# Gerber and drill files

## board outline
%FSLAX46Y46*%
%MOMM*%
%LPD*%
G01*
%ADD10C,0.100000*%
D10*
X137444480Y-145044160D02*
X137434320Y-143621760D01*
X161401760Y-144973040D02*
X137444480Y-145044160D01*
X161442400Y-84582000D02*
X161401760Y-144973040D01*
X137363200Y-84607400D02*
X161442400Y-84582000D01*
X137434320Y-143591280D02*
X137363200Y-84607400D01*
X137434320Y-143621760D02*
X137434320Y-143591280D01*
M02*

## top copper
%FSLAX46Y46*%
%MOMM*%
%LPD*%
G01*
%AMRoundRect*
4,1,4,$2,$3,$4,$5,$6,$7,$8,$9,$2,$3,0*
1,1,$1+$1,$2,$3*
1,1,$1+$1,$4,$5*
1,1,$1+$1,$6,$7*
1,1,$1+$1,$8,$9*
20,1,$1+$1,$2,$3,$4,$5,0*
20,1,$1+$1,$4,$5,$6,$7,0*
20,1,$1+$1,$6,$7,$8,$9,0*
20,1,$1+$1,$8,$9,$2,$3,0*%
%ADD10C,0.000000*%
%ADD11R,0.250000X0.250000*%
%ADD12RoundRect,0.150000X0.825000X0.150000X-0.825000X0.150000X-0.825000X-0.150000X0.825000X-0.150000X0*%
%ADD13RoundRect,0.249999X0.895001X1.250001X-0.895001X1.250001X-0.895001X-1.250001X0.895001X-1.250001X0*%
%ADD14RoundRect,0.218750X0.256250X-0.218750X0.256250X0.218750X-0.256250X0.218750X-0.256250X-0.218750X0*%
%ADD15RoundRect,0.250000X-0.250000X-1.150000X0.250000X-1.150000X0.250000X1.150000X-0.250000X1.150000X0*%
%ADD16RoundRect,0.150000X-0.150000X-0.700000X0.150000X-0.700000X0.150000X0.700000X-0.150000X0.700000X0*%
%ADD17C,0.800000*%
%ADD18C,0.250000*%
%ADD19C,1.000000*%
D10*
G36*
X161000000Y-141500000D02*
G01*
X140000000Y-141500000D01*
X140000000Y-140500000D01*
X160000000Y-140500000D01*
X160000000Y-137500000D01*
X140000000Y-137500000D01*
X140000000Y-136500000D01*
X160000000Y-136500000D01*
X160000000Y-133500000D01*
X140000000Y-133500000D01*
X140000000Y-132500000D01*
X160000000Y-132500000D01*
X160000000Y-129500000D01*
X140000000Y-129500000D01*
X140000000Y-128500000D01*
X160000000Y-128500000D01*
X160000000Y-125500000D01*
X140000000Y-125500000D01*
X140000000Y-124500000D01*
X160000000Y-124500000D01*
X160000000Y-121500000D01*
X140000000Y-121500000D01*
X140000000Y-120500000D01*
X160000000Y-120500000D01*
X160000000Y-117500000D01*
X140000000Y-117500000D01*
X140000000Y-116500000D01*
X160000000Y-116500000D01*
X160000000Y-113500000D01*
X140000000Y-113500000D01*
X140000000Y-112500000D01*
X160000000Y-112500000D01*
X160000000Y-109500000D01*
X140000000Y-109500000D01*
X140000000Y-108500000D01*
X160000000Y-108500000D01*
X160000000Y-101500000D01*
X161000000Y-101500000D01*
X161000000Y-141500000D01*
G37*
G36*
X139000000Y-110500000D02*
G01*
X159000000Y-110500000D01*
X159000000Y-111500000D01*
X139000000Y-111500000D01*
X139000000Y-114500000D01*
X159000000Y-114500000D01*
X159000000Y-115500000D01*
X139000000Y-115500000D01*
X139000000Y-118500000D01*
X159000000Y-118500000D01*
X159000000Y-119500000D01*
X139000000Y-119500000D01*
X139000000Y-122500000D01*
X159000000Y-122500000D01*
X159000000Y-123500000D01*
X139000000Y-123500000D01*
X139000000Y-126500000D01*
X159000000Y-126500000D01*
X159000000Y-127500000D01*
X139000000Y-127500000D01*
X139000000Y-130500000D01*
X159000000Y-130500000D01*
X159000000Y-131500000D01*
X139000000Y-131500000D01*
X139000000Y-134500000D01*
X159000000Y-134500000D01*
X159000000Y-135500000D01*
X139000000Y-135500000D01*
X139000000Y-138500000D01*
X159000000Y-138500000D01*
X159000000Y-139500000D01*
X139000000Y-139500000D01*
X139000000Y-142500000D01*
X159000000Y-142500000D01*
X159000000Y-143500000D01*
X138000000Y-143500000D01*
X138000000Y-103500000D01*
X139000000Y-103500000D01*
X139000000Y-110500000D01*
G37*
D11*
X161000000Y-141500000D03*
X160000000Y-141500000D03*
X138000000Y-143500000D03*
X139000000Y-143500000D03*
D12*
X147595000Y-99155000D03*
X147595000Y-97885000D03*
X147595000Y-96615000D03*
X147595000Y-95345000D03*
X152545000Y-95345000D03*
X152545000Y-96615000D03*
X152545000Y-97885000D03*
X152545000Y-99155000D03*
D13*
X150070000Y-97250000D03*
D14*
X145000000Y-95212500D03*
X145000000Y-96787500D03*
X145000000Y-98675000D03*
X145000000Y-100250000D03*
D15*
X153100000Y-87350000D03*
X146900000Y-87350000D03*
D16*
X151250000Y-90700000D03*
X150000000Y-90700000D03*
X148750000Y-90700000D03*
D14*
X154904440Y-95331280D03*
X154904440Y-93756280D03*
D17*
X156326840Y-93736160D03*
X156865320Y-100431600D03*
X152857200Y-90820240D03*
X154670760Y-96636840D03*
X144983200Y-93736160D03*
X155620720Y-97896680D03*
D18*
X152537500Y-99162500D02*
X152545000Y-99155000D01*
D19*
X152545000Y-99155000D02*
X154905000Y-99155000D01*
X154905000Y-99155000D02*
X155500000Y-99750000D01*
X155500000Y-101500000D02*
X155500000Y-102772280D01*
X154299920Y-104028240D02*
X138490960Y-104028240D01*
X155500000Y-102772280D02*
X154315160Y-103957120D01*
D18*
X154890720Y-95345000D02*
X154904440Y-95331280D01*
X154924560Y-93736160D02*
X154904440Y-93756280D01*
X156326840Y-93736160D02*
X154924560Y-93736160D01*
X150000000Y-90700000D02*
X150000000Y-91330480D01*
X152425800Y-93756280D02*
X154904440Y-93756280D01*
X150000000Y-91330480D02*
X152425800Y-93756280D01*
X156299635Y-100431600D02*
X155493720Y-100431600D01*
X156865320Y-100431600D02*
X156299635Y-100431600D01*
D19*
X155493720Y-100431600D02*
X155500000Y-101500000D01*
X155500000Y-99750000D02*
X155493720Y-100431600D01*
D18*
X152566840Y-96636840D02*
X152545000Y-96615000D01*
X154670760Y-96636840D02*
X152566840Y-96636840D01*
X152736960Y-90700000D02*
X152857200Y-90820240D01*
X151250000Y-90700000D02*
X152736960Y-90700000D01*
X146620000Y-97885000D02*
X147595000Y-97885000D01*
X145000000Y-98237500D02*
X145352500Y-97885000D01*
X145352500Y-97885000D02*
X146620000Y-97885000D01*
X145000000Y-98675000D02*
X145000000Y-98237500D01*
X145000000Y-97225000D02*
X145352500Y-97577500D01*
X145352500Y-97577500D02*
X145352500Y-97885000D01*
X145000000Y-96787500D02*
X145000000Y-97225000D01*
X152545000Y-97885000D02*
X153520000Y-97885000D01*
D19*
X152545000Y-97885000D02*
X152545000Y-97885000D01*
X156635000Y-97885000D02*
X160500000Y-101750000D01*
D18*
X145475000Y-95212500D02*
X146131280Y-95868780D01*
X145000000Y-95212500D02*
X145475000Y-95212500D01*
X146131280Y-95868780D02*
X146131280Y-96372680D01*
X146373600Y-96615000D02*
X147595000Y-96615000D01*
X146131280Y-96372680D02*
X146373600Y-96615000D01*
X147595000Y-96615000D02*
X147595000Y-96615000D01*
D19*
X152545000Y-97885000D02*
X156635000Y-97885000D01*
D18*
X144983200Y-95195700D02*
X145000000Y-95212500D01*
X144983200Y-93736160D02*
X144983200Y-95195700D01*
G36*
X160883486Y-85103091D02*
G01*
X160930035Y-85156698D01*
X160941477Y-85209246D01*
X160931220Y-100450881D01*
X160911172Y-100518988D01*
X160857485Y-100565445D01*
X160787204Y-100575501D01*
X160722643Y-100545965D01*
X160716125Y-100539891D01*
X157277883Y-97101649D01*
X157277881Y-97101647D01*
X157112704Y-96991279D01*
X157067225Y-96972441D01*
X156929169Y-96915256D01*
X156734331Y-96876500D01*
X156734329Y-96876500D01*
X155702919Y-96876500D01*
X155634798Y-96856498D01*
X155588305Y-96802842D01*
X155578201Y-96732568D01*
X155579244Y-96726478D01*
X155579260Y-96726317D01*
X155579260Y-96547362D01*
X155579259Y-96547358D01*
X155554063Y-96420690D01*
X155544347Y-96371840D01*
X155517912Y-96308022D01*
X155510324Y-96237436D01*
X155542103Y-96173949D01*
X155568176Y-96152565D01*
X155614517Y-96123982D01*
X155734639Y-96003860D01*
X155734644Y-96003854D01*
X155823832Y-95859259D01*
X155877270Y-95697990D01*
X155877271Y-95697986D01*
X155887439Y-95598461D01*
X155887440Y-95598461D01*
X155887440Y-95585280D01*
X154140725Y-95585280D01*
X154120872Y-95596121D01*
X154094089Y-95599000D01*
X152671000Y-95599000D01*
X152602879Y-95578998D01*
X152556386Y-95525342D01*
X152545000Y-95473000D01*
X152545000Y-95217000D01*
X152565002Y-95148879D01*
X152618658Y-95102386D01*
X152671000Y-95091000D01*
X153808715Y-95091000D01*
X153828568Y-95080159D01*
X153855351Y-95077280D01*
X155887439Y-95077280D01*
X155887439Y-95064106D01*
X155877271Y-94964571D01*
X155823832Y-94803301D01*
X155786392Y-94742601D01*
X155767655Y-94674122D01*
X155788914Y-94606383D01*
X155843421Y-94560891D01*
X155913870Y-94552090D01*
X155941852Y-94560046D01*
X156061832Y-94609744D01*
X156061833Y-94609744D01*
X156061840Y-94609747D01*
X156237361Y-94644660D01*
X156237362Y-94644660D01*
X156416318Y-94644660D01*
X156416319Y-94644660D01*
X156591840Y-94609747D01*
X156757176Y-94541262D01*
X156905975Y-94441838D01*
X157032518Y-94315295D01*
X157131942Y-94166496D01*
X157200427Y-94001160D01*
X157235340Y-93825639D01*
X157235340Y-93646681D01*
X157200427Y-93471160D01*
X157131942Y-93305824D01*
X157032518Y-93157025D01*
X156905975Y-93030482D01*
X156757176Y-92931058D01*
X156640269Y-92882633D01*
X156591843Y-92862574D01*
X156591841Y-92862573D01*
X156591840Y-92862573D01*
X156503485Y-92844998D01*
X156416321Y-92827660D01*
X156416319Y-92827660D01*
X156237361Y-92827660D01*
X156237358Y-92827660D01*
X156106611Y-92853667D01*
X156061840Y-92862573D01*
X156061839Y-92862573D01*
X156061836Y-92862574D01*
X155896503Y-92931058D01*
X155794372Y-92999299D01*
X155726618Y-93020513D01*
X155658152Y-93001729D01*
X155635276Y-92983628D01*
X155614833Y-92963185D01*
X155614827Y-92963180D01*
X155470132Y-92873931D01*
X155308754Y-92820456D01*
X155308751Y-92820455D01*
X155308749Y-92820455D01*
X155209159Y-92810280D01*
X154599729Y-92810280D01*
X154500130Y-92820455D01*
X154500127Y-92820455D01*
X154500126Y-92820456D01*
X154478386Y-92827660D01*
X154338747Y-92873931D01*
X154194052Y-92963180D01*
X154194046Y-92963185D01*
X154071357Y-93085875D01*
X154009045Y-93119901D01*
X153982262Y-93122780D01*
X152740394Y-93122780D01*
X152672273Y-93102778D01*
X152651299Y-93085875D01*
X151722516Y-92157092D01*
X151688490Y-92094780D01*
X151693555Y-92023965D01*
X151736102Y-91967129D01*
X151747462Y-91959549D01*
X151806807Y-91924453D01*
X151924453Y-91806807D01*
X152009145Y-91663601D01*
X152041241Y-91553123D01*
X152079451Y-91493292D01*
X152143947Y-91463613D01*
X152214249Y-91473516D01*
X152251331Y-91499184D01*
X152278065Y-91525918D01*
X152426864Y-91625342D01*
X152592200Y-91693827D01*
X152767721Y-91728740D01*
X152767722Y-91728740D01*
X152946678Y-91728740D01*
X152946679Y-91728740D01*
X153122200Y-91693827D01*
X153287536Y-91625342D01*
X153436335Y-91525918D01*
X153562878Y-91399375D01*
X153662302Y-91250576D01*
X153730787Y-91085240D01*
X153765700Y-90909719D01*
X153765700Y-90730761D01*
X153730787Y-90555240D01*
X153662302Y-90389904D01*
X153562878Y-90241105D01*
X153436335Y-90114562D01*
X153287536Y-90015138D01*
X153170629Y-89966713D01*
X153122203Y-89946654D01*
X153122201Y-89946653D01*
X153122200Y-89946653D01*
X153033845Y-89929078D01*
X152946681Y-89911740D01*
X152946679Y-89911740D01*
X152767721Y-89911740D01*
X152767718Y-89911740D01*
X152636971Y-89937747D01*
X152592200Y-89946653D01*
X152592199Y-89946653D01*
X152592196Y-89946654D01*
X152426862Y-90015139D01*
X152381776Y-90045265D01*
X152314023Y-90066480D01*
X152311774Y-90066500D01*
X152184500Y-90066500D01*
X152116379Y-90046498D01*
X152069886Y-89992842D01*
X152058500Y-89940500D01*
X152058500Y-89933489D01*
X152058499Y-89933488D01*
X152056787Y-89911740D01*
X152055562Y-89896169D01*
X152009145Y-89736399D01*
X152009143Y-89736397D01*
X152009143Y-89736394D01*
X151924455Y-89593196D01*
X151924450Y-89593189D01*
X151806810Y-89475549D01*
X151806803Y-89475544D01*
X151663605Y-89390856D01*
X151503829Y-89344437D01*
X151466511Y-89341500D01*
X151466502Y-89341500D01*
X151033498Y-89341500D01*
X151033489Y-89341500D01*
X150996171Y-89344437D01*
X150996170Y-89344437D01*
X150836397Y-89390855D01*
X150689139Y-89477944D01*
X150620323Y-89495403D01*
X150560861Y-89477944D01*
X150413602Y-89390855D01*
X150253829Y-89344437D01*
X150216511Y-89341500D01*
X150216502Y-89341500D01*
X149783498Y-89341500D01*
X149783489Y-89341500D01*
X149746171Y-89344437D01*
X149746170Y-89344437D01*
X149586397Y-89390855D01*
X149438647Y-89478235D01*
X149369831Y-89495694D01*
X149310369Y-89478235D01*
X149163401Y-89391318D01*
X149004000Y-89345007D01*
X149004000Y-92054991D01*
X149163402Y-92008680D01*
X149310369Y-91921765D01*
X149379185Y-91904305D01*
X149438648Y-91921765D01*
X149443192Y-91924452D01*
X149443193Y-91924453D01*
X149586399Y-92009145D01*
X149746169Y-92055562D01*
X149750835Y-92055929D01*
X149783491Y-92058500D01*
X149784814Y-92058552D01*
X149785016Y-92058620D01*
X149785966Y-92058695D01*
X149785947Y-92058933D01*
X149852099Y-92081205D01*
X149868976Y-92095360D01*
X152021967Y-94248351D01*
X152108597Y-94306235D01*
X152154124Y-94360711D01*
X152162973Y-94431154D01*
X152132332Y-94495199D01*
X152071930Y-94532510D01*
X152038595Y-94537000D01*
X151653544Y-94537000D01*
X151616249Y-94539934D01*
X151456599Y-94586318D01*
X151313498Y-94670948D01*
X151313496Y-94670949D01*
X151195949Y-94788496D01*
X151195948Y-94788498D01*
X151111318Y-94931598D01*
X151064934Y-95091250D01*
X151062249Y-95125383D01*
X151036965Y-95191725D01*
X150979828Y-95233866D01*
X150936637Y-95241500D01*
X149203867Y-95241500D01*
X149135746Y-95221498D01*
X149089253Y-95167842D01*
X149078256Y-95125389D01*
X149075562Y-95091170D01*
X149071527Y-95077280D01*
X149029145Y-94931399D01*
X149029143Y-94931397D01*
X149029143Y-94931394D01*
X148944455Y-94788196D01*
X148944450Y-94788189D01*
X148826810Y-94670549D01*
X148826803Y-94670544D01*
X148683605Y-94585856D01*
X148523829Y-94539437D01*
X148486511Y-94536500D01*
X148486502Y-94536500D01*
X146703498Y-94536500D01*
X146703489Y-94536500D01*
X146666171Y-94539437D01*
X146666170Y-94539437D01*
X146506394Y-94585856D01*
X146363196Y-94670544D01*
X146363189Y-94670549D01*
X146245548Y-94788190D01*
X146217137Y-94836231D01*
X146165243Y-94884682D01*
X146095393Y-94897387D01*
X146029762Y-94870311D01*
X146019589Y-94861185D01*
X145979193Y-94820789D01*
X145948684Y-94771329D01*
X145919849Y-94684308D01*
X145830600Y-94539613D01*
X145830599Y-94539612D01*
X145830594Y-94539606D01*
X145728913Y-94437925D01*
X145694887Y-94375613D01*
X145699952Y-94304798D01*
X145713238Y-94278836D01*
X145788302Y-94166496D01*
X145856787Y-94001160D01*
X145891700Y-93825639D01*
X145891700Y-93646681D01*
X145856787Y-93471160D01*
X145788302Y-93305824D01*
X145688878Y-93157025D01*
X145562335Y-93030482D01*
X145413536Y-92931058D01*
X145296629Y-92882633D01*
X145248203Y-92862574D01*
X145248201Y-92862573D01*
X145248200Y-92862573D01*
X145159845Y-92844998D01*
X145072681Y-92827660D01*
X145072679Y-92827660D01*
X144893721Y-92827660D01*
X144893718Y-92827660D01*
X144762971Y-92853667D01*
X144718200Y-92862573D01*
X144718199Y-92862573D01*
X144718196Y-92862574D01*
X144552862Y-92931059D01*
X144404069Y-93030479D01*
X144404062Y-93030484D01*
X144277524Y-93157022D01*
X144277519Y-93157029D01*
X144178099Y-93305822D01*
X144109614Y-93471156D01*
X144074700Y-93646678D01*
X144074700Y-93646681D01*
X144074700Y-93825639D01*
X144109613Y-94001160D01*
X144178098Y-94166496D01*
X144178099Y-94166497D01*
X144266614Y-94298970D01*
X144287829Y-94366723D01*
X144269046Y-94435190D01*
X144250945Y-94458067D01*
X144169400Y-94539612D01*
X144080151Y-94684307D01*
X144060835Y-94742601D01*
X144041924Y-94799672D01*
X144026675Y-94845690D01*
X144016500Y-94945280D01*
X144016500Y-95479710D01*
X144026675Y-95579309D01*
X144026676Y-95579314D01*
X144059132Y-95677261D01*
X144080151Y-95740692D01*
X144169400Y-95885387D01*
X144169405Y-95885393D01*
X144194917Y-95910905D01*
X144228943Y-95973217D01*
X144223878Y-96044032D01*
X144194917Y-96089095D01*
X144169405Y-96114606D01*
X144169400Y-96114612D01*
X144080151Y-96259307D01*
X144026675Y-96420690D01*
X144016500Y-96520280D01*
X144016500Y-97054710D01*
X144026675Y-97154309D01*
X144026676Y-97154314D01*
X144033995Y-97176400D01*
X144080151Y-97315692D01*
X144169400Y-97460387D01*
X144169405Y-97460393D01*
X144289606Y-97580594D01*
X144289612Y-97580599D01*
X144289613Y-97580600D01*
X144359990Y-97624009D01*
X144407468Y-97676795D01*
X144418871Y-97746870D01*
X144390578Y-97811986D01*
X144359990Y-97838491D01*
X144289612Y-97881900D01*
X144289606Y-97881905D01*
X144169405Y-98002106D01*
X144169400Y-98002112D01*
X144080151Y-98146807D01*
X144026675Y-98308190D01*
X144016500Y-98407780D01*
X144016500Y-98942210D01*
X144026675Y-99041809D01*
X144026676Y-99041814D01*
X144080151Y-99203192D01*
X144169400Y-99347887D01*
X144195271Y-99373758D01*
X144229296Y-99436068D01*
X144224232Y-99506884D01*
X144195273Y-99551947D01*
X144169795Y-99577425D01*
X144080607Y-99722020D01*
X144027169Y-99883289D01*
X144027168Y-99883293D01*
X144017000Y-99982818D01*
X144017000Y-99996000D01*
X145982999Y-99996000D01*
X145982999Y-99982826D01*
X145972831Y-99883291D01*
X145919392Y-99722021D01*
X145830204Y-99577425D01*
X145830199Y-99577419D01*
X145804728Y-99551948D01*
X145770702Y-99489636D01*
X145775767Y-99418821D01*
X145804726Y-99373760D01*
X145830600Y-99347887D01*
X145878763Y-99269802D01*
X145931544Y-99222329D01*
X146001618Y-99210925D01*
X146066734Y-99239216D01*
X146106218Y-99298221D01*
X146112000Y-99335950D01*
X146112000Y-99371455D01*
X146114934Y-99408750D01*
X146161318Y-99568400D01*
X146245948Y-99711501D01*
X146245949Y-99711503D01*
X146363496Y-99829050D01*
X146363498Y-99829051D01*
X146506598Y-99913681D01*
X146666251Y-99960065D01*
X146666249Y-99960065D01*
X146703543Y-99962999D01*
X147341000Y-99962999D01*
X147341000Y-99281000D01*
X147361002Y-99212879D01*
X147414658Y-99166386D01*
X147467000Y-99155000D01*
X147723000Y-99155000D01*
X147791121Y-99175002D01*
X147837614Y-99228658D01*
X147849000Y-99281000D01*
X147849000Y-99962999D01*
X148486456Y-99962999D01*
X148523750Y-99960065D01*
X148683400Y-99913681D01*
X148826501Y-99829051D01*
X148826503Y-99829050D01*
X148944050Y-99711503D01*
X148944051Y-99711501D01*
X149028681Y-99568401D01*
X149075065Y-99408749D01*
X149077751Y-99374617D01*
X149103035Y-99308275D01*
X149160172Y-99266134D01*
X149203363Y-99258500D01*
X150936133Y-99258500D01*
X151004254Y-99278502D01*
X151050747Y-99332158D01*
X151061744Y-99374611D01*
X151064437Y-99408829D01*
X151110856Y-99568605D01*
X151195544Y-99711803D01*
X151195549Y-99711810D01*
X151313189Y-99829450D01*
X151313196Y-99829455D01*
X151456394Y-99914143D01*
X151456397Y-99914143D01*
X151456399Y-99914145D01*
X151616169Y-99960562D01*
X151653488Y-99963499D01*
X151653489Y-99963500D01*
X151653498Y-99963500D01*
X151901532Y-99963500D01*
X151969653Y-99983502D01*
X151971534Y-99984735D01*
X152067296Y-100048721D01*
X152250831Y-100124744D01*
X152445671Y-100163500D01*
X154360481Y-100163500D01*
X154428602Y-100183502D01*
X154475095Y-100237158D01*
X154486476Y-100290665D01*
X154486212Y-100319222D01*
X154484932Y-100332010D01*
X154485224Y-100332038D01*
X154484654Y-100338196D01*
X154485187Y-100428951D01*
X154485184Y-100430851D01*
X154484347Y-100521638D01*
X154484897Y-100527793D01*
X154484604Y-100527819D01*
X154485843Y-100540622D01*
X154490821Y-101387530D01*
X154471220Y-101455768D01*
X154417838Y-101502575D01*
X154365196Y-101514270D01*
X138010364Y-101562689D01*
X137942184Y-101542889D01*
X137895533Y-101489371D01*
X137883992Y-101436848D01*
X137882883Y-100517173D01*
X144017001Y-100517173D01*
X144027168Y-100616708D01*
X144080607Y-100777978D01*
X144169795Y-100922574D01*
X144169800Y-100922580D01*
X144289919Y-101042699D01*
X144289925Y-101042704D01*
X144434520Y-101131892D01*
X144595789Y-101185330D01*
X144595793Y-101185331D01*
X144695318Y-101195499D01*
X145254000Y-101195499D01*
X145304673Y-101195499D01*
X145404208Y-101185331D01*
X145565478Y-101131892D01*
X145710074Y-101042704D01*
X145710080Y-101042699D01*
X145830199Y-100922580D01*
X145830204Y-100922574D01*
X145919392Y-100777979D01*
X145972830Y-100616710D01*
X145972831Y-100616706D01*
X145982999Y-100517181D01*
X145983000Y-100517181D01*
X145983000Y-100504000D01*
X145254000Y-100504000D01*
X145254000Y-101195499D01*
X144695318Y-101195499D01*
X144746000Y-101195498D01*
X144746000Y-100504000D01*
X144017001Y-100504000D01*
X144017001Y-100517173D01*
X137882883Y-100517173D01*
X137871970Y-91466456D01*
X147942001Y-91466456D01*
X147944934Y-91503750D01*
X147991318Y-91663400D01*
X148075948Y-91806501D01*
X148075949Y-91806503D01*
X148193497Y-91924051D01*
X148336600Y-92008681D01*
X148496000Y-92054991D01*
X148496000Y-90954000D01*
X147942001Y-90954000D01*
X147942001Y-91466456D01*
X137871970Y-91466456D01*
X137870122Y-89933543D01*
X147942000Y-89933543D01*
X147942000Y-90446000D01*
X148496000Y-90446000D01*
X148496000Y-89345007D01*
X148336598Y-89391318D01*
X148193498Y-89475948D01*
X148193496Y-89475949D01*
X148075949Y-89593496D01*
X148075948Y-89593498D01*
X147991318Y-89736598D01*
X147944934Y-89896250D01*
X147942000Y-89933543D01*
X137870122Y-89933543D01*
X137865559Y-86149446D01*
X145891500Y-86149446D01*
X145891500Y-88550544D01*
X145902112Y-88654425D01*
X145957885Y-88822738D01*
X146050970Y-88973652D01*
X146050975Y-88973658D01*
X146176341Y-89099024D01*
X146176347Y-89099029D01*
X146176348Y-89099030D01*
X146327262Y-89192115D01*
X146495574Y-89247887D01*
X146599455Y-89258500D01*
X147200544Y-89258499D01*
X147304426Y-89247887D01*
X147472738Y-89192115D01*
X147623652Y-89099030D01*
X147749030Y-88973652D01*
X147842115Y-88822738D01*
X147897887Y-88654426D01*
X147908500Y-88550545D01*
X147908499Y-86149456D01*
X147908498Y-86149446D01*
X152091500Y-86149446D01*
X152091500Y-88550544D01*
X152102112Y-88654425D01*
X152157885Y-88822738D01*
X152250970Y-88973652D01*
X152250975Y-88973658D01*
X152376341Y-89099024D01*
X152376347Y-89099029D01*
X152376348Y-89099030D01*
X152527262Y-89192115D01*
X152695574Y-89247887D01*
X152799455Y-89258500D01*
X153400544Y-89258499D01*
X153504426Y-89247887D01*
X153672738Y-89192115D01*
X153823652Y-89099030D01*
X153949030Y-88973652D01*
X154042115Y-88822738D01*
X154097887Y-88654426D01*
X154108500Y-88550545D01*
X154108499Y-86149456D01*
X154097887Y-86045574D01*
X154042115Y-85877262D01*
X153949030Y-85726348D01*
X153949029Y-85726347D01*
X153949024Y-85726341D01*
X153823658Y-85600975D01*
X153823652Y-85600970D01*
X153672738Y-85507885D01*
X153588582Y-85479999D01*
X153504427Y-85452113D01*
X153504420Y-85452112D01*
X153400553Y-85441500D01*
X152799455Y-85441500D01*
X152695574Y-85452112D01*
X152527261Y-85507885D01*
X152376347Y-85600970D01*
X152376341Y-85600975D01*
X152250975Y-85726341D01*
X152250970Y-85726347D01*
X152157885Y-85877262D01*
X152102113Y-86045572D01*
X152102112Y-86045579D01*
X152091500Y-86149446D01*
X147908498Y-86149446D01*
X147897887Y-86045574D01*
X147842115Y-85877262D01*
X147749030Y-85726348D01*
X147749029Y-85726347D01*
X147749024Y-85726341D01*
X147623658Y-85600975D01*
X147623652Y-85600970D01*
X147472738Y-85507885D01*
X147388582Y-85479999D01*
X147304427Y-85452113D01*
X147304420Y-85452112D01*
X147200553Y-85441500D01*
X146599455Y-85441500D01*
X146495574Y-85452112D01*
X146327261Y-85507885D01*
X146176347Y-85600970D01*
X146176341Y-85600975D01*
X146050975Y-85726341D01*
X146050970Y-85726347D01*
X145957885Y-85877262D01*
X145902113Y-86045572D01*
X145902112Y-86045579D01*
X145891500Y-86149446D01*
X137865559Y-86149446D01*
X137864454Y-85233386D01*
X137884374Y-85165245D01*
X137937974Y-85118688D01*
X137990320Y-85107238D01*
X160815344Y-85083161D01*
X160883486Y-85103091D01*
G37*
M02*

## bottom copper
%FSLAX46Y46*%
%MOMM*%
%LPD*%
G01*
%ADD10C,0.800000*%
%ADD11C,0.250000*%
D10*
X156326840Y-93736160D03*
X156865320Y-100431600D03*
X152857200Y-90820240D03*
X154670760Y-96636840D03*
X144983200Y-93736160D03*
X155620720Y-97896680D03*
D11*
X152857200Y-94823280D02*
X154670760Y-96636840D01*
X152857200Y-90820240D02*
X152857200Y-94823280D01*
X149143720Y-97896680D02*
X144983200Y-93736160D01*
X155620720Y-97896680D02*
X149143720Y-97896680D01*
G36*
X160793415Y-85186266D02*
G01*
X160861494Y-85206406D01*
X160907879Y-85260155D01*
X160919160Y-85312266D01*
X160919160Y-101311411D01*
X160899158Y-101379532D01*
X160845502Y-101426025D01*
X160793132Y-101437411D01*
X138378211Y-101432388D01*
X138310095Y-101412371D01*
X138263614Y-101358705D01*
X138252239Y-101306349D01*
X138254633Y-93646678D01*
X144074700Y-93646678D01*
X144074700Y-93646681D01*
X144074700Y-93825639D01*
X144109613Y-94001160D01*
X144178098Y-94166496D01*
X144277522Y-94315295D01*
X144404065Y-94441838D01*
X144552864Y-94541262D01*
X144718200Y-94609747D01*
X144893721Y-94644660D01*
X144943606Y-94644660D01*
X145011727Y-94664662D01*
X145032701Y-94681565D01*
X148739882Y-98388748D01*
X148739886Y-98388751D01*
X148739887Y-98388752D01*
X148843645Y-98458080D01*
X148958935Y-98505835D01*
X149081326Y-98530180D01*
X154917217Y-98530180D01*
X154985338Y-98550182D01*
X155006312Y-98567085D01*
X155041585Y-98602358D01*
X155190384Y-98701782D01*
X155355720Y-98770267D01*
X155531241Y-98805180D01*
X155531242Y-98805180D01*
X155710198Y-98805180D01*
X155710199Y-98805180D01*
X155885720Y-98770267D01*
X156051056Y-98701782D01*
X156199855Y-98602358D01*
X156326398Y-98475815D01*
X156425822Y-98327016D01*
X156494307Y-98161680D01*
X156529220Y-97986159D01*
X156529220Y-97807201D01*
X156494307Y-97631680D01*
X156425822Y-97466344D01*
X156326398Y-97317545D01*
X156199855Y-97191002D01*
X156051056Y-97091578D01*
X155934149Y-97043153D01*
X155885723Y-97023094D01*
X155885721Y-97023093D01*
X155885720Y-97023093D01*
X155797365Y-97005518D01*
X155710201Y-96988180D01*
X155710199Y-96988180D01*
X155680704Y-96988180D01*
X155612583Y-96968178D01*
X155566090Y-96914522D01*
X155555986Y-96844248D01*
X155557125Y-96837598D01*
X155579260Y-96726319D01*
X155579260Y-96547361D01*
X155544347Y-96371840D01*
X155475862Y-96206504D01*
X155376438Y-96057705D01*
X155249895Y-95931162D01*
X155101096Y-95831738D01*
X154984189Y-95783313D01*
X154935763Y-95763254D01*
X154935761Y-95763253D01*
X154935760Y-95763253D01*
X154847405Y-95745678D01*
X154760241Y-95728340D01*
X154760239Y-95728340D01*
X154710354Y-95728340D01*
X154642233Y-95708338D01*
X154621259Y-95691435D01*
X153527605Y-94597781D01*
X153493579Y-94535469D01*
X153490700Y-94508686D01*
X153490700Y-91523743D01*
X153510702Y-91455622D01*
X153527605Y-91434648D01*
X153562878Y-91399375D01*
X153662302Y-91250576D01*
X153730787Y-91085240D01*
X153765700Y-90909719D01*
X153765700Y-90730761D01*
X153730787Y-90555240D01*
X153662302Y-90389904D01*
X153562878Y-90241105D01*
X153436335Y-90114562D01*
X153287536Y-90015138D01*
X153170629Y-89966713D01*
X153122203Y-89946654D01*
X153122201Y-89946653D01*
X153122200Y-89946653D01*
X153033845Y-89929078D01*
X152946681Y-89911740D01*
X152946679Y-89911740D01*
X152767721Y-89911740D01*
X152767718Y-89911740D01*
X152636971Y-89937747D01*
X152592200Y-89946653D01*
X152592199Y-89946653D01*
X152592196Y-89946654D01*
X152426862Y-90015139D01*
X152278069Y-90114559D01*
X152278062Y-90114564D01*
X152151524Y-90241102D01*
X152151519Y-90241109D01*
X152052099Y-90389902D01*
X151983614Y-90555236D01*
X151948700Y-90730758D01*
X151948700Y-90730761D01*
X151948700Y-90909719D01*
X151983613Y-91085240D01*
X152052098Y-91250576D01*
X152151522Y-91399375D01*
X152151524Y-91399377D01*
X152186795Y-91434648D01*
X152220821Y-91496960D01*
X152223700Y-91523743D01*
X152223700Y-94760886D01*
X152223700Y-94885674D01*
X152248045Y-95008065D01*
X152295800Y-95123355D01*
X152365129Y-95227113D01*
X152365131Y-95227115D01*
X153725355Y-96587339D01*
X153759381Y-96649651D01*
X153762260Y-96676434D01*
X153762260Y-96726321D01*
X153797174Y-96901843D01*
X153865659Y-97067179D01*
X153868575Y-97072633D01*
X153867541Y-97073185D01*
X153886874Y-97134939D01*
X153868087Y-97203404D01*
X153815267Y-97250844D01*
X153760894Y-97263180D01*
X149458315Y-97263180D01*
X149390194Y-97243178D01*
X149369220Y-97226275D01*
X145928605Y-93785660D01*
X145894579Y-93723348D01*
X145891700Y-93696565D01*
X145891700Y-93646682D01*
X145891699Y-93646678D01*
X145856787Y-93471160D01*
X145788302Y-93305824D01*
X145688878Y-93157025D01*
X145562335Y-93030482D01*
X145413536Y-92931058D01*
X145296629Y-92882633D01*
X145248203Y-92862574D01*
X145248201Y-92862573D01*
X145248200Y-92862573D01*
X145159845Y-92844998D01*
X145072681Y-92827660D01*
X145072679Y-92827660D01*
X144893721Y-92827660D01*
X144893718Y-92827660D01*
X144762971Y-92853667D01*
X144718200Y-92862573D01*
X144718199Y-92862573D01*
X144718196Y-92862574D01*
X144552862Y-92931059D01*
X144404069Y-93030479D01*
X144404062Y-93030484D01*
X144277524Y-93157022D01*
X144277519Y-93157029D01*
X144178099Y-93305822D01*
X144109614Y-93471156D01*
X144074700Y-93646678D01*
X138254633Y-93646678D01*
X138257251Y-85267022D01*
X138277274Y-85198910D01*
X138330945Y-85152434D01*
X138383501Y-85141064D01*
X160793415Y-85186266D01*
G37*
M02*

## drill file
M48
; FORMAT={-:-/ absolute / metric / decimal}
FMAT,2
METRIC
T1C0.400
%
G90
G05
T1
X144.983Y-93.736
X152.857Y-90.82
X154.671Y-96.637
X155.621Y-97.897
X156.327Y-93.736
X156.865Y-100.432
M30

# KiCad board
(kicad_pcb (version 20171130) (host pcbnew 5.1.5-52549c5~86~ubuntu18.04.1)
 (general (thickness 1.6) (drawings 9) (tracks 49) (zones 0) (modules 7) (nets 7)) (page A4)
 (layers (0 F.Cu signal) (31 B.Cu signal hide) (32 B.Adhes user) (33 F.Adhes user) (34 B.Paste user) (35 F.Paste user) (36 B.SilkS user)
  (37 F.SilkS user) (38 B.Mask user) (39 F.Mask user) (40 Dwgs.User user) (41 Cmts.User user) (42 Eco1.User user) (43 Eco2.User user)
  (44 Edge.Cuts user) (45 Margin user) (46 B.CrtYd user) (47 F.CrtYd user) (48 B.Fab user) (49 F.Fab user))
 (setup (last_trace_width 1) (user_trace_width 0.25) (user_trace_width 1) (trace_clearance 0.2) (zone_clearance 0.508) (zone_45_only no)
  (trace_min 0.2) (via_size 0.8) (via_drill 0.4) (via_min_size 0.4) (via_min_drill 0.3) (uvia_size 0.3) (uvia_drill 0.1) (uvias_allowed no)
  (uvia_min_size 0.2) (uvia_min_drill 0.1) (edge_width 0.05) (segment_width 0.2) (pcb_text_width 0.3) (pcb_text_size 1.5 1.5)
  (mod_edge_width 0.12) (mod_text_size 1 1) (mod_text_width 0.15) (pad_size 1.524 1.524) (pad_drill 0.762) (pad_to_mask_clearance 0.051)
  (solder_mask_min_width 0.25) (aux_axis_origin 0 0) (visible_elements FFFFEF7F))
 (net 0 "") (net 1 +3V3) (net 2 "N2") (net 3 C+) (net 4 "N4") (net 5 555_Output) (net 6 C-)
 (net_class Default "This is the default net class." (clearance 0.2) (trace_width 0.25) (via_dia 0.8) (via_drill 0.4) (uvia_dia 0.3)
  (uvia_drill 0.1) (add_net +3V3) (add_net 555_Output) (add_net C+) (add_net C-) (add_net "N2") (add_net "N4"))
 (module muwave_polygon (layer F.Cu) (at 160.5 141.5 180)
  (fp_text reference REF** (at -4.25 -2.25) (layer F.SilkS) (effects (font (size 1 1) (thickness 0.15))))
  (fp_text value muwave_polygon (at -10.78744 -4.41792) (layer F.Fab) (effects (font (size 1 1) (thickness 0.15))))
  (fp_poly
   (pts (xy -0.5 0) (xy 20.5 0) (xy 20.5 1) (xy 0.5 1) (xy 0.5 4) (xy 20.5 4) (xy 20.5 5) (xy 0.5 5) (xy 0.5 8) (xy 20.5 8) (xy 20.5 9)
    (xy 0.5 9) (xy 0.5 12) (xy 20.5 12) (xy 20.5 13) (xy 0.5 13) (xy 0.5 16) (xy 20.5 16) (xy 20.5 17) (xy 0.5 17) (xy 0.5 20) (xy 20.5 20)
    (xy 20.5 21) (xy 0.5 21) (xy 0.5 24) (xy 20.5 24) (xy 20.5 25) (xy 0.5 25) (xy 0.5 28) (xy 20.5 28) (xy 20.5 29) (xy 0.5 29) (xy 0.5 32)
    (xy 20.5 32) (xy 20.5 33) (xy 0.5 33) (xy 0.5 40) (xy -0.5 40) (xy -0.5 0))
   (layer F.Cu) (width 0))
  (pad 2 smd rect (at -0.5 0 180) (size 0.25 0.25) (layers F.Cu))
  (pad 1 smd rect (at 0.5 0 180) (size 0.25 0.25) (layers F.Cu)))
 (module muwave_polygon (layer F.Cu) (at 138.5 143.5)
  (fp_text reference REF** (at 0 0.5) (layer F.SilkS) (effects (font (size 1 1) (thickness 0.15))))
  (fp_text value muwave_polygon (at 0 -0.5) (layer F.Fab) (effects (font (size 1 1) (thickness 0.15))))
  (fp_poly
   (pts (xy -0.5 0) (xy 20.5 0) (xy 20.5 -1) (xy 0.5 -1) (xy 0.5 -4) (xy 20.5 -4) (xy 20.5 -5) (xy 0.5 -5) (xy 0.5 -8) (xy 20.5 -8)
    (xy 20.5 -9) (xy 0.5 -9) (xy 0.5 -12) (xy 20.5 -12) (xy 20.5 -13) (xy 0.5 -13) (xy 0.5 -16) (xy 20.5 -16) (xy 20.5 -17) (xy 0.5 -17)
    (xy 0.5 -20) (xy 20.5 -20) (xy 20.5 -21) (xy 0.5 -21) (xy 0.5 -24) (xy 20.5 -24) (xy 20.5 -25) (xy 0.5 -25) (xy 0.5 -28) (xy 20.5 -28)
    (xy 20.5 -29) (xy 0.5 -29) (xy 0.5 -32) (xy 20.5 -32) (xy 20.5 -33) (xy 0.5 -33) (xy 0.5 -40) (xy -0.5 -40) (xy -0.5 0))
   (layer F.Cu) (width 0))
  (pad 2 smd rect (at -0.5 0) (size 0.25 0.25) (layers F.Cu)) (pad 1 smd rect (at 0.5 0) (size 0.25 0.25) (layers F.Cu)))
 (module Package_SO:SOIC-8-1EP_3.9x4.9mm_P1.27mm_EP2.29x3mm (layer F.Cu) (at 150.07 97.25 180)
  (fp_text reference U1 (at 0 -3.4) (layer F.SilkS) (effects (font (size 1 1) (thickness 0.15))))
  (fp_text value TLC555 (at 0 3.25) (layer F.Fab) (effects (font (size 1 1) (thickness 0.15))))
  (pad 8 smd roundrect (at 2.475 -1.905 180) (size 1.95 0.6) (layers F.Cu F.Paste F.Mask) (roundrect_rratio 0.25) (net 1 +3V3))
  (pad 7 smd roundrect (at 2.475 -0.635 180) (size 1.95 0.6) (layers F.Cu F.Paste F.Mask) (roundrect_rratio 0.25) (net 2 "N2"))
  (pad 6 smd roundrect (at 2.475 0.635 180) (size 1.95 0.6) (layers F.Cu F.Paste F.Mask) (roundrect_rratio 0.25) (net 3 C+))
  (pad 5 smd roundrect (at 2.475 1.905 180) (size 1.95 0.6) (layers F.Cu F.Paste F.Mask) (roundrect_rratio 0.25) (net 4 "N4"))
  (pad 4 smd roundrect (at -2.475 1.905 180) (size 1.95 0.6) (layers F.Cu F.Paste F.Mask) (roundrect_rratio 0.25) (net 1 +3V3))
  (pad 3 smd roundrect (at -2.475 0.635 180) (size 1.95 0.6) (layers F.Cu F.Paste F.Mask) (roundrect_rratio 0.25) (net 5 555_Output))
  (pad 2 smd roundrect (at -2.475 -0.635 180) (size 1.95 0.6) (layers F.Cu F.Paste F.Mask) (roundrect_rratio 0.25) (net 3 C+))
  (pad 1 smd roundrect (at -2.475 -1.905 180) (size 1.95 0.6) (layers F.Cu F.Paste F.Mask) (roundrect_rratio 0.25) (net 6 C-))
  (pad "" smd roundrect (at 0.57 0.75 180) (size 0.92 1.21) (layers F.Paste) (roundrect_rratio 0.25))
  (pad "" smd roundrect (at 0.57 -0.75 180) (size 0.92 1.21) (layers F.Paste) (roundrect_rratio 0.25))
  (pad "" smd roundrect (at -0.57 0.75 180) (size 0.92 1.21) (layers F.Paste) (roundrect_rratio 0.25))
  (pad "" smd roundrect (at -0.57 -0.75 180) (size 0.92 1.21) (layers F.Paste) (roundrect_rratio 0.25))
  (pad 9 smd roundrect (at 0 0 180) (size 2.29 3) (layers F.Cu F.Mask) (roundrect_rratio 0.10917)))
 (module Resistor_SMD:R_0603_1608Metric (layer F.Cu) (at 145 96 90)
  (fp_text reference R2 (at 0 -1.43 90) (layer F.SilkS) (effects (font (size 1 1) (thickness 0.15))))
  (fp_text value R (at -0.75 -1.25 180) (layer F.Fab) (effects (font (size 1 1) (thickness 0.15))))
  (pad 2 smd roundrect (at 0.7875 0 90) (size 0.875 0.95) (layers F.Cu F.Paste F.Mask) (roundrect_rratio 0.25) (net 3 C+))
  (pad 1 smd roundrect (at -0.7875 0 90) (size 0.875 0.95) (layers F.Cu F.Paste F.Mask) (roundrect_rratio 0.25) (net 2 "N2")))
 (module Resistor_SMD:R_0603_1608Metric (layer F.Cu) (at 145 99.4625 90)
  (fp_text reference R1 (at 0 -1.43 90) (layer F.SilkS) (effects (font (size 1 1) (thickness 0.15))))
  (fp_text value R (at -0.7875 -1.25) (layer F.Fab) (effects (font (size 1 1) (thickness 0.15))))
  (pad 2 smd roundrect (at 0.7875 0 90) (size 0.875 0.95) (layers F.Cu F.Paste F.Mask) (roundrect_rratio 0.25) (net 2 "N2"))
  (pad 1 smd roundrect (at -0.7875 0 90) (size 0.875 0.95) (layers F.Cu F.Paste F.Mask) (roundrect_rratio 0.25) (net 1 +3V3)))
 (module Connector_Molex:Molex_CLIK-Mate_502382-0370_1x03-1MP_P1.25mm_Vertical (layer F.Cu) (at 150 88.75)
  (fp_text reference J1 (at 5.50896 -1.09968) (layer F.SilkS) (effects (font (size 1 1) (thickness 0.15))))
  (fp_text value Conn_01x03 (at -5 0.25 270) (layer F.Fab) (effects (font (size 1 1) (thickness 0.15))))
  (pad MP smd roundrect (at 3.1 -1.4) (size 1 2.8) (layers F.Cu F.Paste F.Mask) (roundrect_rratio 0.25))
  (pad MP smd roundrect (at -3.1 -1.4) (size 1 2.8) (layers F.Cu F.Paste F.Mask) (roundrect_rratio 0.25))
  (pad 3 smd roundrect (at 1.25 1.95) (size 0.6 1.7) (layers F.Cu F.Paste F.Mask) (roundrect_rratio 0.25) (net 5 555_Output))
  (pad 2 smd roundrect (at 0 1.95) (size 0.6 1.7) (layers F.Cu F.Paste F.Mask) (roundrect_rratio 0.25) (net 6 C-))
  (pad 1 smd roundrect (at -1.25 1.95) (size 0.6 1.7) (layers F.Cu F.Paste F.Mask) (roundrect_rratio 0.25) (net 1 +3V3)))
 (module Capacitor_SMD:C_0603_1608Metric (layer F.Cu) (at 154.90444 94.54378 90)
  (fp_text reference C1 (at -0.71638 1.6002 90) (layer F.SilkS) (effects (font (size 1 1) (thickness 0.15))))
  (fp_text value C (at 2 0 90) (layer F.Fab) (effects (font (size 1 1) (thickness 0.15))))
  (pad 1 smd roundrect (at -0.7875 0 90) (size 0.875 0.95) (layers F.Cu F.Paste F.Mask) (roundrect_rratio 0.25) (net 1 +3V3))
  (pad 2 smd roundrect (at 0.7875 0 90) (size 0.875 0.95) (layers F.Cu F.Paste F.Mask) (roundrect_rratio 0.25) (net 6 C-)))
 (gr_line (start 137.44448 145.04416) (end 137.43432 143.62176) (layer Edge.Cuts) (width 0.1))
 (gr_line (start 161.40176 144.97304) (end 137.44448 145.04416) (layer Edge.Cuts) (width 0.1))
 (gr_line (start 161.4424 84.582) (end 161.40176 144.97304) (layer Edge.Cuts) (width 0.1))
 (gr_line (start 137.3632 84.6074) (end 161.4424 84.582) (layer Edge.Cuts) (width 0.1))
 (gr_line (start 137.43432 143.59128) (end 137.3632 84.6074) (layer Edge.Cuts) (width 0.1))
 (gr_line (start 137.43432 143.62176) (end 137.43432 143.59128) (layer Edge.Cuts) (width 0.1))
 (segment (start 152.5375 99.1625) (end 152.545 99.155) (width 0.25) (layer F.Cu) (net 6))
 (segment (start 152.545 99.155) (end 154.905 99.155) (width 1) (layer F.Cu) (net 6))
 (segment (start 154.905 99.155) (end 155.5 99.75) (width 1) (layer F.Cu) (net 6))
 (segment (start 155.5 101.5) (end 155.5 102.77228) (width 1) (layer F.Cu) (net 6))
 (segment (start 154.29992 104.02824) (end 138.49096 104.02824) (width 1) (layer F.Cu) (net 6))
 (segment (start 155.5 102.77228) (end 154.31516 103.95712) (width 1) (layer F.Cu) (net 6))
 (segment (start 154.89072 95.345) (end 154.90444 95.33128) (width 0.25) (layer F.Cu) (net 1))
 (via (at 156.32684 93.73616) (size 0.8) (drill 0.4) (layers F.Cu B.Cu) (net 6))
 (segment (start 154.92456 93.73616) (end 154.90444 93.75628) (width 0.25) (layer F.Cu) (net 6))
 (segment (start 156.32684 93.73616) (end 154.92456 93.73616) (width 0.25) (layer F.Cu) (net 6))
 (segment (start 150 90.7) (end 150 91.33048) (width 0.25) (layer F.Cu) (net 6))
 (segment (start 152.4258 93.75628) (end 154.90444 93.75628) (width 0.25) (layer F.Cu) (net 6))
 (segment (start 150 91.33048) (end 152.4258 93.75628) (width 0.25) (layer F.Cu) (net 6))
 (via (at 156.86532 100.4316) (size 0.8) (drill 0.4) (layers F.Cu B.Cu) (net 6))
 (segment (start 156.299635 100.4316) (end 155.49372 100.4316) (width 0.25) (layer F.Cu) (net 6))
 (segment (start 156.86532 100.4316) (end 156.299635 100.4316) (width 0.25) (layer F.Cu) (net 6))
 (segment (start 155.49372 100.4316) (end 155.5 101.5) (width 1) (layer F.Cu) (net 6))
 (segment (start 155.5 99.75) (end 155.49372 100.4316) (width 1) (layer F.Cu) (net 6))
 (via (at 152.8572 90.82024) (size 0.8) (drill 0.4) (layers F.Cu B.Cu) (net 5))
 (via (at 154.67076 96.63684) (size 0.8) (drill 0.4) (layers F.Cu B.Cu) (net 5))
 (segment (start 152.56684 96.63684) (end 152.545 96.615) (width 0.25) (layer F.Cu) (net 5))
 (segment (start 154.67076 96.63684) (end 152.56684 96.63684) (width 0.25) (layer F.Cu) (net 5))
 (segment (start 152.73696 90.7) (end 152.8572 90.82024) (width 0.25) (layer F.Cu) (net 5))
 (segment (start 151.25 90.7) (end 152.73696 90.7) (width 0.25) (layer F.Cu) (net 5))
 (segment (start 152.8572 94.82328) (end 154.67076 96.63684) (width 0.25) (layer B.Cu) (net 5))
 (segment (start 152.8572 90.82024) (end 152.8572 94.82328) (width 0.25) (layer B.Cu) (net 5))
 (segment (start 146.62 97.885) (end 147.595 97.885) (width 0.25) (layer F.Cu) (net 2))
 (segment (start 145 98.2375) (end 145.3525 97.885) (width 0.25) (layer F.Cu) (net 2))
 (segment (start 145.3525 97.885) (end 146.62 97.885) (width 0.25) (layer F.Cu) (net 2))
 (segment (start 145 98.675) (end 145 98.2375) (width 0.25) (layer F.Cu) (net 2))
 (segment (start 145 97.225) (end 145.3525 97.5775) (width 0.25) (layer F.Cu) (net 2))
 (segment (start 145.3525 97.5775) (end 145.3525 97.885) (width 0.25) (layer F.Cu) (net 2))
 (segment (start 145 96.7875) (end 145 97.225) (width 0.25) (layer F.Cu) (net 2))
 (segment (start 152.545 97.885) (end 153.52 97.885) (width 0.25) (layer F.Cu) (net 3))
 (segment (start 152.545 97.885) (end 152.545 97.885) (width 1) (layer F.Cu) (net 3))
 (segment (start 156.635 97.885) (end 160.5 101.75) (width 1) (layer F.Cu) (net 3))
 (segment (start 145.475 95.2125) (end 146.13128 95.86878) (width 0.25) (layer F.Cu) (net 3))
 (segment (start 145 95.2125) (end 145.475 95.2125) (width 0.25) (layer F.Cu) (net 3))
 (segment (start 146.13128 95.86878) (end 146.13128 96.37268) (width 0.25) (layer F.Cu) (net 3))
 (segment (start 146.3736 96.615) (end 147.595 96.615) (width 0.25) (layer F.Cu) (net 3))
 (segment (start 146.13128 96.37268) (end 146.3736 96.615) (width 0.25) (layer F.Cu) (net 3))
 (segment (start 147.595 96.615) (end 147.595 96.615) (width 0.25) (layer F.Cu) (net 3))
 (via (at 144.9832 93.73616) (size 0.8) (drill 0.4) (layers F.Cu B.Cu) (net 3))
 (segment (start 152.545 97.885) (end 156.635 97.885) (width 1) (layer F.Cu) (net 3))
 (via (at 155.62072 97.89668) (size 0.8) (drill 0.4) (layers F.Cu B.Cu) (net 3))
 (segment (start 144.9832 95.1957) (end 145 95.2125) (width 0.25) (layer F.Cu) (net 3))
 (segment (start 144.9832 93.73616) (end 144.9832 95.1957) (width 0.25) (layer F.Cu) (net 3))
 (segment (start 149.14372 97.89668) (end 144.9832 93.73616) (width 0.25) (layer B.Cu) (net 3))
 (segment (start 155.62072 97.89668) (end 149.14372 97.89668) (width 0.25) (layer B.Cu) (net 3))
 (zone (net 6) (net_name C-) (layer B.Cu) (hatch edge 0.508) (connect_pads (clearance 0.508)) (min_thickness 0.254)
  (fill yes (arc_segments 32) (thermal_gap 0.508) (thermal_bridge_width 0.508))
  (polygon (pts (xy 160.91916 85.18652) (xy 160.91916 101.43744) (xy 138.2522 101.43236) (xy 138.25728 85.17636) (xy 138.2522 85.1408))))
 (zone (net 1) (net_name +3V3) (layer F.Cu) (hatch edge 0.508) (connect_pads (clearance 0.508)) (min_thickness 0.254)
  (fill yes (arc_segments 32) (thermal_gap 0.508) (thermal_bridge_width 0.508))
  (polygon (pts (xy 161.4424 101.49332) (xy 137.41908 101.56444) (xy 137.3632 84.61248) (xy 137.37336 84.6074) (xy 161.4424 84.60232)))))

